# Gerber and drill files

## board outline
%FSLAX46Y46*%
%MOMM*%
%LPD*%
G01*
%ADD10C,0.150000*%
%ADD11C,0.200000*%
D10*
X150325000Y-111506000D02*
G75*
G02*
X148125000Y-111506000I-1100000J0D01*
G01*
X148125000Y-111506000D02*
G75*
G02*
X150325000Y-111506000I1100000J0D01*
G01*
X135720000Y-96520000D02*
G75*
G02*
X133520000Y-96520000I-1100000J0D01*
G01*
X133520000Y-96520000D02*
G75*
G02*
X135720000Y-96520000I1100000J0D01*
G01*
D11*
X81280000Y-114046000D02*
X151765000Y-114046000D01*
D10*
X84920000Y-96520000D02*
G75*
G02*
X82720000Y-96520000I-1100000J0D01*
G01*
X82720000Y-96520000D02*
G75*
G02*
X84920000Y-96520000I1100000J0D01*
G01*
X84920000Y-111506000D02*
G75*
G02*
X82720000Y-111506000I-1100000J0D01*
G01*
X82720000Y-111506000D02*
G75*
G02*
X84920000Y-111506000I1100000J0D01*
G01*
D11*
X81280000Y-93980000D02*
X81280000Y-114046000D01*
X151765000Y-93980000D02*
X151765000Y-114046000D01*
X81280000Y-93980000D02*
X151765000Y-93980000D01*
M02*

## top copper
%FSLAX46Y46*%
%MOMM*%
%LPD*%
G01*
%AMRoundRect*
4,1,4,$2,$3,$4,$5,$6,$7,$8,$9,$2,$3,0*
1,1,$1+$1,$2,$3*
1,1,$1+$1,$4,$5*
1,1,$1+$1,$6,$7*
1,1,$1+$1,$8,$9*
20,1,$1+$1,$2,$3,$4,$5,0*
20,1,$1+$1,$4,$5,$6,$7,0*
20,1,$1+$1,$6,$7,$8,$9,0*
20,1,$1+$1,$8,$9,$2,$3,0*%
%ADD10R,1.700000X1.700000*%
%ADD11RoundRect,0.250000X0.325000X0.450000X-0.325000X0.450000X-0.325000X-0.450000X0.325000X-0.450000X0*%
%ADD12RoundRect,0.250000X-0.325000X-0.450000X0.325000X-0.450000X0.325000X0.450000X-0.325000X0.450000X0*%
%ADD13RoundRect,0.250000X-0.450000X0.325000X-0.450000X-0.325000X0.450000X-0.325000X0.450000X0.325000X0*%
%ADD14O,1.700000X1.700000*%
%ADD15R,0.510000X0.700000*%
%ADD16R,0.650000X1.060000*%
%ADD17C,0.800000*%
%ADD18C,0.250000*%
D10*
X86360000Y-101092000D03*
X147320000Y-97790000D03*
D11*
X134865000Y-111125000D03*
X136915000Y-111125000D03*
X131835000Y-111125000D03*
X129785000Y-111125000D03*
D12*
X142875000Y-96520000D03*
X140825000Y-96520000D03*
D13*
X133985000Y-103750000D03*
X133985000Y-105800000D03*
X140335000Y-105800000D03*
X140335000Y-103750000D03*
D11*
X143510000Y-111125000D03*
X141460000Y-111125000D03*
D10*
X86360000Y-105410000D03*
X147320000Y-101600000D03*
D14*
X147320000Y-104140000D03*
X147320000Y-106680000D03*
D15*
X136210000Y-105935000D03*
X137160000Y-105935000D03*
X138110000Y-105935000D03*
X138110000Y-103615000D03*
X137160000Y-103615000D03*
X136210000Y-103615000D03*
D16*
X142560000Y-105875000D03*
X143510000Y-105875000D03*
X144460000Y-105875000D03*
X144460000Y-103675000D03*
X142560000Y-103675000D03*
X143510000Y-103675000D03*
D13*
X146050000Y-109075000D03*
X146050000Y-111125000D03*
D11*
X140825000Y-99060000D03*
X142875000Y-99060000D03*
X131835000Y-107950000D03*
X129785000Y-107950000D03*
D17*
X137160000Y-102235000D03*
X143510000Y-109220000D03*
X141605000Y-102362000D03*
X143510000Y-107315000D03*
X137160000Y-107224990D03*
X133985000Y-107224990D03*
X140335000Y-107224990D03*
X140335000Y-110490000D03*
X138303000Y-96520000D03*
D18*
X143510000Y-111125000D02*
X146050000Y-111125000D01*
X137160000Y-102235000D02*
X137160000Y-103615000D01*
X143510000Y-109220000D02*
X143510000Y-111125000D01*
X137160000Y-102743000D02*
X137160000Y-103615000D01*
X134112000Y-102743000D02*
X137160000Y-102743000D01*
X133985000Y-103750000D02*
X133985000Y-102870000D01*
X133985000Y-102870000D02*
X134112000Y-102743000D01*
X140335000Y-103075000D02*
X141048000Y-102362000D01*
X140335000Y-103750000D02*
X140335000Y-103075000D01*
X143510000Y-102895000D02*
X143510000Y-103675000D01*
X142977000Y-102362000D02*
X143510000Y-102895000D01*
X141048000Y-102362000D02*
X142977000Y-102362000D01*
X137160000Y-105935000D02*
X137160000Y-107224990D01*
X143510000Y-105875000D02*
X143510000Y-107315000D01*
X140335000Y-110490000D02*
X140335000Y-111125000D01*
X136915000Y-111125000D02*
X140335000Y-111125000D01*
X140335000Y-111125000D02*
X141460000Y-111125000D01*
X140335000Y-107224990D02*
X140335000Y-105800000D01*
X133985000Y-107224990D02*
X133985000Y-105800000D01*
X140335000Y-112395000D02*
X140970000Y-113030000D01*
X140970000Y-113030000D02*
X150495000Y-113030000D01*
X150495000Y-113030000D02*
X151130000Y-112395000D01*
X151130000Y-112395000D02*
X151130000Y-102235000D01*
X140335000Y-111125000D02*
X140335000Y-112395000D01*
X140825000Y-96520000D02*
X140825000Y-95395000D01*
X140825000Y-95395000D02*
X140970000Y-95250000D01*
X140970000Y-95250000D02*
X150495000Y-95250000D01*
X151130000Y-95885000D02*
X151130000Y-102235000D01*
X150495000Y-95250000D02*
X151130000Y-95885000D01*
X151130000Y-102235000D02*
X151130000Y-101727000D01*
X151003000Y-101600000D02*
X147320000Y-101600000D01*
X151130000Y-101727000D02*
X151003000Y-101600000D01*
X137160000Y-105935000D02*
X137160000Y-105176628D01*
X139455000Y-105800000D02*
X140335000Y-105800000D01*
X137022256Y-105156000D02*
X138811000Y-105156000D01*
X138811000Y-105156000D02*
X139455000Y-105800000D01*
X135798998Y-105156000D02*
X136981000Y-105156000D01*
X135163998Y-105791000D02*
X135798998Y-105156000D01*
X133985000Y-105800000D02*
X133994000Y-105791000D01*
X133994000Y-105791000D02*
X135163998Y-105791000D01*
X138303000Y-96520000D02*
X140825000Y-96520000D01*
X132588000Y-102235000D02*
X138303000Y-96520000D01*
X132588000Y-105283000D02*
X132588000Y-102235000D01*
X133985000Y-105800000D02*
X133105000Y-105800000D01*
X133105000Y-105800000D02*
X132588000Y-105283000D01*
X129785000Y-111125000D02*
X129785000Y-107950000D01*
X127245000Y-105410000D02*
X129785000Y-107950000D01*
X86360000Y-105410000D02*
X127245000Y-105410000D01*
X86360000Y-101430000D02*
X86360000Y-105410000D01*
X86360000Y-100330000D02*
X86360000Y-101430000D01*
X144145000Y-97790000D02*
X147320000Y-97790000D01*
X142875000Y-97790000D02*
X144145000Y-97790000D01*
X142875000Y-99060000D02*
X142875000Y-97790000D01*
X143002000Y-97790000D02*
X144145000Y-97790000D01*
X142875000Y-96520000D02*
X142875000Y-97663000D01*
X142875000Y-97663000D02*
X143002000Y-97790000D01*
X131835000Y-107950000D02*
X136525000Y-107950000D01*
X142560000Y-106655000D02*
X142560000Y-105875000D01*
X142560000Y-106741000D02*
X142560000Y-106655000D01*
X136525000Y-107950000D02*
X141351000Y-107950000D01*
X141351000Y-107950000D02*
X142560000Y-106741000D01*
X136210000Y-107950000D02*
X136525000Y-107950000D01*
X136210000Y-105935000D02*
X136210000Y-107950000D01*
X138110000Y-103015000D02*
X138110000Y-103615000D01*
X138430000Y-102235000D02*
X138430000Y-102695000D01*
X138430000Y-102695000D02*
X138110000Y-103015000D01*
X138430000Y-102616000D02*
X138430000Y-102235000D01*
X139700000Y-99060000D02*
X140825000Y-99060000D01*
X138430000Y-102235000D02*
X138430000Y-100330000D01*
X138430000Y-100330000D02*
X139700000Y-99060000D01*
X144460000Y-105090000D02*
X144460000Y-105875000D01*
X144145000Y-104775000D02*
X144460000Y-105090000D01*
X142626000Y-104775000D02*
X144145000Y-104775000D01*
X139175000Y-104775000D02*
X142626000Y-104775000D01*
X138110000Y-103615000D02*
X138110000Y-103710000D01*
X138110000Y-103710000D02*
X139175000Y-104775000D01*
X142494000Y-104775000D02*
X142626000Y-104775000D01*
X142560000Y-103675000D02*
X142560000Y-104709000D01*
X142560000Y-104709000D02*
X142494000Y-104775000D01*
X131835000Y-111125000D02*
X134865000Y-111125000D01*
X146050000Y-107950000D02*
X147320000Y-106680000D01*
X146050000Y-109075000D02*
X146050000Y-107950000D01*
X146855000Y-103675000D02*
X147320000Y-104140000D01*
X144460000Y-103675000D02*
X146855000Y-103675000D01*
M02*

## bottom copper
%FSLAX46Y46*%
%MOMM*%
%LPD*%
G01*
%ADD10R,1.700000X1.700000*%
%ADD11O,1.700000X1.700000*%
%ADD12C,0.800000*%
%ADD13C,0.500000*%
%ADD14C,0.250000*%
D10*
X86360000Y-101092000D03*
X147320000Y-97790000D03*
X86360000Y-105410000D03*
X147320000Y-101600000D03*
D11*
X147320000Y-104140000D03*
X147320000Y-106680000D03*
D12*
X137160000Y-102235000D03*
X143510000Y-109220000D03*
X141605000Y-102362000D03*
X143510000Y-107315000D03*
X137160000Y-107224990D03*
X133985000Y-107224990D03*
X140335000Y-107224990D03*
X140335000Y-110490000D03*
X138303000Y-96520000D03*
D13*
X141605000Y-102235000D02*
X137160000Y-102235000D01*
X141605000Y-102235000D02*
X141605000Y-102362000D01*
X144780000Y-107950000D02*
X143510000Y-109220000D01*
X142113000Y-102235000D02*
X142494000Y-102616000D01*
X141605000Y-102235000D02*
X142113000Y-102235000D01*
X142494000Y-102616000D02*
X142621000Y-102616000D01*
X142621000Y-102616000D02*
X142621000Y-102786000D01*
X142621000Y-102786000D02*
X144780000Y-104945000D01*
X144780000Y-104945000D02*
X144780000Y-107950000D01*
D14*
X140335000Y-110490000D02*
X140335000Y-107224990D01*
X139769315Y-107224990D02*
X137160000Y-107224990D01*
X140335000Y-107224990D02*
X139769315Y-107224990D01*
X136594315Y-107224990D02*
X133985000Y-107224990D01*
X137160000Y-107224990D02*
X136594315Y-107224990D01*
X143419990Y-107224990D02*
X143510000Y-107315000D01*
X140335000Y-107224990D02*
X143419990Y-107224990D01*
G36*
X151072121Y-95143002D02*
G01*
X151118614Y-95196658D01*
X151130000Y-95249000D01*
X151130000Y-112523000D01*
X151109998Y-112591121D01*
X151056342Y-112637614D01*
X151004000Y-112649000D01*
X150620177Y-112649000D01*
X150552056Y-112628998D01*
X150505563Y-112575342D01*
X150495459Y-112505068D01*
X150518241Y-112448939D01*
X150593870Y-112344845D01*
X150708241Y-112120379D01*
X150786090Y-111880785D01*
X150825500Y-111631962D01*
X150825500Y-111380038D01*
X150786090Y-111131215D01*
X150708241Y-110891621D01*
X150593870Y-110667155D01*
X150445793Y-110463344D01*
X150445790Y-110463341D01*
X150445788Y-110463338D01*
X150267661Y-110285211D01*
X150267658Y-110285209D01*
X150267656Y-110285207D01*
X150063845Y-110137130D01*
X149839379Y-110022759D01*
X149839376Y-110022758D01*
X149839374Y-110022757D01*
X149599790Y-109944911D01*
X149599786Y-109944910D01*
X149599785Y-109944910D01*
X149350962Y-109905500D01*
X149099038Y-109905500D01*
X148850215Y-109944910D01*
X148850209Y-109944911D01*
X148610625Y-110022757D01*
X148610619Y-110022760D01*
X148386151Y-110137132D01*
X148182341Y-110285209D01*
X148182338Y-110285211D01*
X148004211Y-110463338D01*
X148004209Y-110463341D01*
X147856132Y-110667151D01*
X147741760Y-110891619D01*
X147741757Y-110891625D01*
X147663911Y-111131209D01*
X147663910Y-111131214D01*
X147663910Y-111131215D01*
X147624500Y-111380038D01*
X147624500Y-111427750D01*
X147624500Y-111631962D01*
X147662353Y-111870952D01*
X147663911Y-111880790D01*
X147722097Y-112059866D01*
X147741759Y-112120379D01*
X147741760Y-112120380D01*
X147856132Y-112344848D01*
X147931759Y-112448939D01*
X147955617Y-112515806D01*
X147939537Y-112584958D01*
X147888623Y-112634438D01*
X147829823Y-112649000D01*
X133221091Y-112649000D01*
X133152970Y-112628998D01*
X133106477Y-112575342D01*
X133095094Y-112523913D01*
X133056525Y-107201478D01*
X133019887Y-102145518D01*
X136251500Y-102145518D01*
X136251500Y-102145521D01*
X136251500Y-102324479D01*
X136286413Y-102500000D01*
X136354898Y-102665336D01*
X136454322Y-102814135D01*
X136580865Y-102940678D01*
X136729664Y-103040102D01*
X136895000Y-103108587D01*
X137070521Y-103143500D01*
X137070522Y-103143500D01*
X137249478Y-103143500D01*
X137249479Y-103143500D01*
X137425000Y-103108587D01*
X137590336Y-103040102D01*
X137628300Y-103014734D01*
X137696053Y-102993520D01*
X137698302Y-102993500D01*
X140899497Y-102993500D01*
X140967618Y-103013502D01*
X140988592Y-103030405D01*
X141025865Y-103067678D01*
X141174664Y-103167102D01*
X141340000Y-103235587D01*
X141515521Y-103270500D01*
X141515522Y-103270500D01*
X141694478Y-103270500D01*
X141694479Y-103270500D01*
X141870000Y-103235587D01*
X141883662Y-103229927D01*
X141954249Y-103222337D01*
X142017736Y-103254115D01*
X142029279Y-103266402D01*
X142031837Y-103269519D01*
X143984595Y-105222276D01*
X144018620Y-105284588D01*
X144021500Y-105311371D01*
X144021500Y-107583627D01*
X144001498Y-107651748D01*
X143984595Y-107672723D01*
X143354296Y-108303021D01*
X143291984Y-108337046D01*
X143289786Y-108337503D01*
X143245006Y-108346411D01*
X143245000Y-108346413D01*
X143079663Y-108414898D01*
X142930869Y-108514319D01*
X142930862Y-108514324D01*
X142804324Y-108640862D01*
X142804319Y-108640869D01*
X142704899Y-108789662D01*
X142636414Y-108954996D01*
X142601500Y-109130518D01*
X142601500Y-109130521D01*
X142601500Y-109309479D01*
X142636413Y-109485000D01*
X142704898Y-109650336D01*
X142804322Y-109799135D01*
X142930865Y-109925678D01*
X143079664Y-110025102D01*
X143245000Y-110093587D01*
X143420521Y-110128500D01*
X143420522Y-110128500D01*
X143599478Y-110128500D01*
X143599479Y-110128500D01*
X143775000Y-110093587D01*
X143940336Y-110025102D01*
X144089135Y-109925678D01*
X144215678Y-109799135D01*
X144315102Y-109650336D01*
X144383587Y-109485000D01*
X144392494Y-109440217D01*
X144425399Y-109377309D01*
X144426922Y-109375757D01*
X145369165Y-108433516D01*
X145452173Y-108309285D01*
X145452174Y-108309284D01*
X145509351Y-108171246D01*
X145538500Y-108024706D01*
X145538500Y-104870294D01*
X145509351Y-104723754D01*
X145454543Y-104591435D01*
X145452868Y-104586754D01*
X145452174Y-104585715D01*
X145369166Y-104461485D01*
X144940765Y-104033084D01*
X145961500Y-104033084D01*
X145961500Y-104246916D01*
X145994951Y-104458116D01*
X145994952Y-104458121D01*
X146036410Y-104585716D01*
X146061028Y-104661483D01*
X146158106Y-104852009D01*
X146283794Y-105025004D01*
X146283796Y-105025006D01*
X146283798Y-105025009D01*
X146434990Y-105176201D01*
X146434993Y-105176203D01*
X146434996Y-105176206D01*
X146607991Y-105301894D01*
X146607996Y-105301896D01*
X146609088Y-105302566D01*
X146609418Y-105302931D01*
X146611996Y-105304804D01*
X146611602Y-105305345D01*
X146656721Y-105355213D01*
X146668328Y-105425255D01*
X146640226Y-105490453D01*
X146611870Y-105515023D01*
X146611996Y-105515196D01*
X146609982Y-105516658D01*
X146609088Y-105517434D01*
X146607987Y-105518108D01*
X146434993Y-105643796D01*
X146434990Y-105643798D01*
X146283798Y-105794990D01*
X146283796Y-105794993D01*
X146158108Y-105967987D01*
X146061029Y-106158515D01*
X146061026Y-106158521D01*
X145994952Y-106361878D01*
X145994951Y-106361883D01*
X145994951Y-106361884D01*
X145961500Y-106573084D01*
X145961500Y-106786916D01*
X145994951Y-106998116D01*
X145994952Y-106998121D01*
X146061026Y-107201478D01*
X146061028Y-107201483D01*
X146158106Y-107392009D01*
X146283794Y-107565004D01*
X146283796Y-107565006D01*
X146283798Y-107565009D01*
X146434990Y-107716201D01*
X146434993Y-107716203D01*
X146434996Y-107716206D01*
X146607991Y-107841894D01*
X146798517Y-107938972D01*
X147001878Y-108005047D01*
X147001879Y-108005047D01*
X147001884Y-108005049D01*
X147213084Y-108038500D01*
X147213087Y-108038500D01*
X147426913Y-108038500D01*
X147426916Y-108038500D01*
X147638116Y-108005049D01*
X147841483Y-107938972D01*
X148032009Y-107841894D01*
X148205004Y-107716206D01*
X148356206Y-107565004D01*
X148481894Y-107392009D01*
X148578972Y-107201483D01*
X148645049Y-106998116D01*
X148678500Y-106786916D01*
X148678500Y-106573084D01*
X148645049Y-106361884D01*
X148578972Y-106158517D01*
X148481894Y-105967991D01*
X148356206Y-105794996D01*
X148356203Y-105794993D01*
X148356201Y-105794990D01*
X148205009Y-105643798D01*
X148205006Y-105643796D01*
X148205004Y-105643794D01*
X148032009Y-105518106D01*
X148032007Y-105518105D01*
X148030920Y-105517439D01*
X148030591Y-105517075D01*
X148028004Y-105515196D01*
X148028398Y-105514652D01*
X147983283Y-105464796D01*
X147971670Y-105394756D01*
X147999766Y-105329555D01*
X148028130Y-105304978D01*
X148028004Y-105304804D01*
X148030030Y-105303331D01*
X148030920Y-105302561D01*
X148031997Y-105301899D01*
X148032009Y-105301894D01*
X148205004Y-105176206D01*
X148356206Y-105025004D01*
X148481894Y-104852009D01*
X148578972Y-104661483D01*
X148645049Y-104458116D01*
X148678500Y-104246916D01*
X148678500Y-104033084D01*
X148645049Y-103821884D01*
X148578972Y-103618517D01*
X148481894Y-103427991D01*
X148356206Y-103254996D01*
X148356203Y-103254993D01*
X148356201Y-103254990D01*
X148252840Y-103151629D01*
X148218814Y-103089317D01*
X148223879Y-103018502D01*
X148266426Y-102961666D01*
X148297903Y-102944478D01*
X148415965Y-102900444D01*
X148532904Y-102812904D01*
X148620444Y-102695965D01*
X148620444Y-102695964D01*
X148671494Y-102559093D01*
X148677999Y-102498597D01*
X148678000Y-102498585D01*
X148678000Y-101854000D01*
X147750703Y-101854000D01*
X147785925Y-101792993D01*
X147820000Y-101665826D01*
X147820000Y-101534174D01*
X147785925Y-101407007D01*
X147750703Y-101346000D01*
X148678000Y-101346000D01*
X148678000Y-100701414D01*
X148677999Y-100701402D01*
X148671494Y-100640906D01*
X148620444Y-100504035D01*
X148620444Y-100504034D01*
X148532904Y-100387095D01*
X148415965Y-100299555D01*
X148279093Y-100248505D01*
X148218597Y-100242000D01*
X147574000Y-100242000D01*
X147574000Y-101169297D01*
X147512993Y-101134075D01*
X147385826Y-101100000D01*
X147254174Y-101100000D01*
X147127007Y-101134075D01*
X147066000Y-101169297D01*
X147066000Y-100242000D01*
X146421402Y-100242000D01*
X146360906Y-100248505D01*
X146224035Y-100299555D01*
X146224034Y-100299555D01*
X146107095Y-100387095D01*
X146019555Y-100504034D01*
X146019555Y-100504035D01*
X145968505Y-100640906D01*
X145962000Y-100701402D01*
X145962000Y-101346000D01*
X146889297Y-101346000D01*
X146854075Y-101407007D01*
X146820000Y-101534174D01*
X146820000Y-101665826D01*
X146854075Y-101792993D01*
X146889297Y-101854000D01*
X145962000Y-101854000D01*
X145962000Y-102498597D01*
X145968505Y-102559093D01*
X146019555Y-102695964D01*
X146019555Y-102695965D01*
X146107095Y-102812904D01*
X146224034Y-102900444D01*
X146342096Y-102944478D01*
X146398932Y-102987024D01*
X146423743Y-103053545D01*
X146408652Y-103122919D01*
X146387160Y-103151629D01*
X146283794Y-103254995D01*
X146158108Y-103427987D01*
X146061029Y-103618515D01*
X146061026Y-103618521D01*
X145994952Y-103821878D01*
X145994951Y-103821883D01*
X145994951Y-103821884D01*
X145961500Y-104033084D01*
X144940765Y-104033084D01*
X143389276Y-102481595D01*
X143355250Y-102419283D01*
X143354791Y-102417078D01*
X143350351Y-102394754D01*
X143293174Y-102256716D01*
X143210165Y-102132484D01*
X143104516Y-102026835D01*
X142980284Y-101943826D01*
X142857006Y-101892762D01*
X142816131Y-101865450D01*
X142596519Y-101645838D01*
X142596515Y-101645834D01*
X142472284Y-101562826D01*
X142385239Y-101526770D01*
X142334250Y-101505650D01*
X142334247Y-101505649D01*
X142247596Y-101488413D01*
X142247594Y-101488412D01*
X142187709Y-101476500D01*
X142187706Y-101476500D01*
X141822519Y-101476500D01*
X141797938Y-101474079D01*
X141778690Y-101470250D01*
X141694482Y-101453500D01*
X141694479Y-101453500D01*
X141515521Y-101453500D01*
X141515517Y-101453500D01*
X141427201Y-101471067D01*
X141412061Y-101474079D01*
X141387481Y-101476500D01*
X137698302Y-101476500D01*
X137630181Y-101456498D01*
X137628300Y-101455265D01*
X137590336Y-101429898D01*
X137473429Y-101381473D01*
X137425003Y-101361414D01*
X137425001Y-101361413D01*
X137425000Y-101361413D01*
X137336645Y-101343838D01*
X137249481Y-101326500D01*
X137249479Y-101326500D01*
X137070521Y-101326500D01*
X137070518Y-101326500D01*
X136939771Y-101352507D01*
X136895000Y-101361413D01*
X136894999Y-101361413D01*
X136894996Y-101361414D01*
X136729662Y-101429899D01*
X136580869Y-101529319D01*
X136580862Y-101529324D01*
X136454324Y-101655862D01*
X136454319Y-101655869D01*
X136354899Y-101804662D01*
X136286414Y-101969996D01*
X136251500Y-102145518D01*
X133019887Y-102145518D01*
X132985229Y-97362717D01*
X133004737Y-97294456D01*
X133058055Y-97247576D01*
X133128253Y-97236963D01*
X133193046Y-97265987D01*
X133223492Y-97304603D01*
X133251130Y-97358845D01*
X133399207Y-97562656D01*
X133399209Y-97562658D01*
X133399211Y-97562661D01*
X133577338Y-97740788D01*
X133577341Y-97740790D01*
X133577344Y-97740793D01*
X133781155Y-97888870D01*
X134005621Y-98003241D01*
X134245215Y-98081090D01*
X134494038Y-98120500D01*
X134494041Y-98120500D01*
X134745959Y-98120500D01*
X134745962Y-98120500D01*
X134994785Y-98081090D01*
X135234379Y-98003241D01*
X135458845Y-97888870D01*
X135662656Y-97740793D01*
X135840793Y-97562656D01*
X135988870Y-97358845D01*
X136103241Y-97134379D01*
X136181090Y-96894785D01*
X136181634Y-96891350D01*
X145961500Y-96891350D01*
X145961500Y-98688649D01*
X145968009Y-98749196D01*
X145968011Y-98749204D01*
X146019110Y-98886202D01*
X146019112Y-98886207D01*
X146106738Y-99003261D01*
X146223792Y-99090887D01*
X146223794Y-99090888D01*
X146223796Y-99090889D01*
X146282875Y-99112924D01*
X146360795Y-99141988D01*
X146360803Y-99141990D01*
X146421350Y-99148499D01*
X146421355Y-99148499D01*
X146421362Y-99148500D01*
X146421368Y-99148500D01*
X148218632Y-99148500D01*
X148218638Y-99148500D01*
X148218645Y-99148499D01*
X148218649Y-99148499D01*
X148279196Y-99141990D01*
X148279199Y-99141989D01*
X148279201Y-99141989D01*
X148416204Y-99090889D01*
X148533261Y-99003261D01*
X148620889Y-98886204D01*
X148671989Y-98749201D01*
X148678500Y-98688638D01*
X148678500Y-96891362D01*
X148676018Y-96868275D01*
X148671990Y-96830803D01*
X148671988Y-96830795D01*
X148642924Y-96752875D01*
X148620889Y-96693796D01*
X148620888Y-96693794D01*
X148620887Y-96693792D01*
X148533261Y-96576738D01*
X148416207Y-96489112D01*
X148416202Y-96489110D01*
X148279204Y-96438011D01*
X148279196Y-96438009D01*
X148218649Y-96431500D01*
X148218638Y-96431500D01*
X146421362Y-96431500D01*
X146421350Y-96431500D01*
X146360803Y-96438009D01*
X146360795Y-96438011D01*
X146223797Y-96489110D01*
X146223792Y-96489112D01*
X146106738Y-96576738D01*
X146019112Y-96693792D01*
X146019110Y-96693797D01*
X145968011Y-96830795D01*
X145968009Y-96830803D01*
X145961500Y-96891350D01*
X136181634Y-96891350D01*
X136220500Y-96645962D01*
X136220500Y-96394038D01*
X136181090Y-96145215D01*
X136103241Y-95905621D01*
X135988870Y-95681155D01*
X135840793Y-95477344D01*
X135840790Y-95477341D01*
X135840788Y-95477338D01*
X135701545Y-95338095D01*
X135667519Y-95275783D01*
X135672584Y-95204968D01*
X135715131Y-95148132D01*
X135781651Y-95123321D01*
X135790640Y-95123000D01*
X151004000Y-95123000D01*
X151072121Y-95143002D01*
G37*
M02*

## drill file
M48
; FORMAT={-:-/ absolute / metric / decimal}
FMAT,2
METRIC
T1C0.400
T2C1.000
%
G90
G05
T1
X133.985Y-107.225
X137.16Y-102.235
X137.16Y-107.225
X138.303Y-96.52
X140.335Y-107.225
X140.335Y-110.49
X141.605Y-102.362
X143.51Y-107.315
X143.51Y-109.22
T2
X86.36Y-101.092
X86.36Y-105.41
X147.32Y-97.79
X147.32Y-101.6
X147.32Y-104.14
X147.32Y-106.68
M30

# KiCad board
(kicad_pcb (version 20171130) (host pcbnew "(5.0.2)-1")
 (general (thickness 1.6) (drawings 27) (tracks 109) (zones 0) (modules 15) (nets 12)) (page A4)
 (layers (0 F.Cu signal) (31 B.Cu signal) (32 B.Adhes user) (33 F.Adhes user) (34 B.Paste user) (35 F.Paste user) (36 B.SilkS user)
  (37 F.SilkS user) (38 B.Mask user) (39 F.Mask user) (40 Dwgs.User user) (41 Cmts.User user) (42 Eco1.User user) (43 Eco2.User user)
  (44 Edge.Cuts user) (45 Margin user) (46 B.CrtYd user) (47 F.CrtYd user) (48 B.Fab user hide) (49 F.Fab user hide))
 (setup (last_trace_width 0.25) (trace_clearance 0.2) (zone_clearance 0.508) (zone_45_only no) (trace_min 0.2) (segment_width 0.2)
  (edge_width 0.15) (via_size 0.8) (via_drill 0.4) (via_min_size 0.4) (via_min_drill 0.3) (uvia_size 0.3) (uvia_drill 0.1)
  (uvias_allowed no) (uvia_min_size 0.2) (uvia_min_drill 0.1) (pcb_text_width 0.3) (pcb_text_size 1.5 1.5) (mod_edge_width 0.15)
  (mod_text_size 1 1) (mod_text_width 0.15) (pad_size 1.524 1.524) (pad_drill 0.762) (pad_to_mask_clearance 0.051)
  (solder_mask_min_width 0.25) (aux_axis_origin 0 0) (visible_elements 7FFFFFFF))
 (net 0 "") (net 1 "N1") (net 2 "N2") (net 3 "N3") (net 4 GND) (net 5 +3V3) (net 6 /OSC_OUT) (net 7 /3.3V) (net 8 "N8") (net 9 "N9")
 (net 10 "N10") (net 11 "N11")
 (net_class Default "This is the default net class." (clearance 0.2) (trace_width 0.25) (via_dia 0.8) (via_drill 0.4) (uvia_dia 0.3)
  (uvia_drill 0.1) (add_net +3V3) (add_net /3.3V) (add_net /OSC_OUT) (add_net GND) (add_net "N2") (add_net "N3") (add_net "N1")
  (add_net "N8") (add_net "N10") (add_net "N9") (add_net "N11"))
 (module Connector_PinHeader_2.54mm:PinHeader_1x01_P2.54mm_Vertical (layer F.Cu) (at 86.36 101.092 180)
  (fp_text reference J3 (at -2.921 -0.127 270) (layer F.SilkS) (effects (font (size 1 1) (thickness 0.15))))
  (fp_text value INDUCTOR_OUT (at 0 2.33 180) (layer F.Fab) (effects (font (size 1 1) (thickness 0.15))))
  (pad 1 thru_hole rect (at 0 0 180) (size 1.7 1.7) (drill 1) (layers *.Cu *.Mask) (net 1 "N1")))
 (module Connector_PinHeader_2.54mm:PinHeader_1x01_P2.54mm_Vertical (layer F.Cu) (at 147.32 97.79)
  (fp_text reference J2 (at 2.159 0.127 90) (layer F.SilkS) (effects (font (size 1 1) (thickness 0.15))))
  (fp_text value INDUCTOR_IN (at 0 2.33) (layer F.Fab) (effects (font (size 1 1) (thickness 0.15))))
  (pad 1 thru_hole rect (at 0 0) (size 1.7 1.7) (drill 1) (layers *.Cu *.Mask) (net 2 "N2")))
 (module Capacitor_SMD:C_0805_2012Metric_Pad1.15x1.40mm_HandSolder (layer F.Cu) (at 135.89 111.125 180)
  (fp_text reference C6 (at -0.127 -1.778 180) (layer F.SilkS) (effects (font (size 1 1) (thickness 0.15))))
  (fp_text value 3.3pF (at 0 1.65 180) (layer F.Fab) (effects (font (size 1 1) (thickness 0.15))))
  (pad 2 smd roundrect (at 1.025 0 180) (size 1.15 1.4) (layers F.Cu F.Paste F.Mask) (roundrect_rratio 0.217391) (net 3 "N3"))
  (pad 1 smd roundrect (at -1.025 0 180) (size 1.15 1.4) (layers F.Cu F.Paste F.Mask) (roundrect_rratio 0.217391) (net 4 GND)))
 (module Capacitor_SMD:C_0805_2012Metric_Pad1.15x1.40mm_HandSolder (layer F.Cu) (at 130.81 111.125 180)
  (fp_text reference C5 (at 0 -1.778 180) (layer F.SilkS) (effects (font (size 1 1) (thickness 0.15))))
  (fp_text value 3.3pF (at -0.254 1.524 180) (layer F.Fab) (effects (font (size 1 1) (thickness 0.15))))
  (pad 1 smd roundrect (at -1.025 0 180) (size 1.15 1.4) (layers F.Cu F.Paste F.Mask) (roundrect_rratio 0.217391) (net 3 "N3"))
  (pad 2 smd roundrect (at 1.025 0 180) (size 1.15 1.4) (layers F.Cu F.Paste F.Mask) (roundrect_rratio 0.217391) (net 1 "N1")))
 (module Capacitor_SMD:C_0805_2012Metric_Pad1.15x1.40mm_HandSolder (layer F.Cu) (at 141.85 96.52)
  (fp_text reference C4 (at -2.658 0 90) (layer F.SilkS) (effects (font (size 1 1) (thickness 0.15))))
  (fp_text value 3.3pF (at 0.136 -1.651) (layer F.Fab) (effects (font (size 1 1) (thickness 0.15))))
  (pad 2 smd roundrect (at 1.025 0) (size 1.15 1.4) (layers F.Cu F.Paste F.Mask) (roundrect_rratio 0.217391) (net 2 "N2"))
  (pad 1 smd roundrect (at -1.025 0) (size 1.15 1.4) (layers F.Cu F.Paste F.Mask) (roundrect_rratio 0.217391) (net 4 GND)))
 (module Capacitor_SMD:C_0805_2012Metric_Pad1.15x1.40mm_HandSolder (layer F.Cu) (at 133.985 104.775 270)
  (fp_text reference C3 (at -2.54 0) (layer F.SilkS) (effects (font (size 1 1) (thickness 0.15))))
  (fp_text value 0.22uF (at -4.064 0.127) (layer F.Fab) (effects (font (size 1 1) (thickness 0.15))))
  (pad 1 smd roundrect (at -1.025 0 270) (size 1.15 1.4) (layers F.Cu F.Paste F.Mask) (roundrect_rratio 0.217391) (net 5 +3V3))
  (pad 2 smd roundrect (at 1.025 0 270) (size 1.15 1.4) (layers F.Cu F.Paste F.Mask) (roundrect_rratio 0.217391) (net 4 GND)))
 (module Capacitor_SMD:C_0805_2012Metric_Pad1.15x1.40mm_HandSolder (layer F.Cu) (at 140.335 104.775 270)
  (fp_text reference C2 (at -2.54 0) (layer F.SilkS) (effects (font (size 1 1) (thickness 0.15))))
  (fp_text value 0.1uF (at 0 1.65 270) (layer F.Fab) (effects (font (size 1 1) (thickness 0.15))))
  (pad 2 smd roundrect (at 1.025 0 270) (size 1.15 1.4) (layers F.Cu F.Paste F.Mask) (roundrect_rratio 0.217391) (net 4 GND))
  (pad 1 smd roundrect (at -1.025 0 270) (size 1.15 1.4) (layers F.Cu F.Paste F.Mask) (roundrect_rratio 0.217391) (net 5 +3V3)))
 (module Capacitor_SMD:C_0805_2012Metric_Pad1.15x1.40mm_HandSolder (layer F.Cu) (at 142.485 111.125 180)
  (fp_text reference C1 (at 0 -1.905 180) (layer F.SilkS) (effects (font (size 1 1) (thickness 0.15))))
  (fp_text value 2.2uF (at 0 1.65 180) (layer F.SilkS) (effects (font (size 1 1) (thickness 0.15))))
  (pad 1 smd roundrect (at -1.025 0 180) (size 1.15 1.4) (layers F.Cu F.Paste F.Mask) (roundrect_rratio 0.217391) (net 5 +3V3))
  (pad 2 smd roundrect (at 1.025 0 180) (size 1.15 1.4) (layers F.Cu F.Paste F.Mask) (roundrect_rratio 0.217391) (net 4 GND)))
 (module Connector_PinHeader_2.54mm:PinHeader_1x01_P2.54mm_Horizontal (layer F.Cu) (at 86.36 105.41 180)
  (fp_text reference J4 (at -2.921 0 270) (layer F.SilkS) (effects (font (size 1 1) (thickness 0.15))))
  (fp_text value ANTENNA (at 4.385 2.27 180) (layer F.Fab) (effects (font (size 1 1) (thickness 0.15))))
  (pad 1 thru_hole rect (at 0 0 180) (size 1.7 1.7) (drill 1) (layers *.Cu *.Mask) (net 1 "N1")))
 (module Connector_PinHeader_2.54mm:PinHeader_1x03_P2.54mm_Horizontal (layer F.Cu) (at 147.32 101.6)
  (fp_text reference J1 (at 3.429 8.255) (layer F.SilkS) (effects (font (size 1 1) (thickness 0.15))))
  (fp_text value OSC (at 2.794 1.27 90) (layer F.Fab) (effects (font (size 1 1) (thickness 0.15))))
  (pad 1 thru_hole rect (at 0 0) (size 1.7 1.7) (drill 1) (layers *.Cu *.Mask) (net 4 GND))
  (pad 2 thru_hole oval (at 0 2.54) (size 1.7 1.7) (drill 1) (layers *.Cu *.Mask) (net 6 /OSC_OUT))
  (pad 3 thru_hole oval (at 0 5.08) (size 1.7 1.7) (drill 1) (layers *.Cu *.Mask) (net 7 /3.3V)))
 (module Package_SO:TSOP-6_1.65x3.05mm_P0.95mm (layer F.Cu) (at 137.16 104.775 90)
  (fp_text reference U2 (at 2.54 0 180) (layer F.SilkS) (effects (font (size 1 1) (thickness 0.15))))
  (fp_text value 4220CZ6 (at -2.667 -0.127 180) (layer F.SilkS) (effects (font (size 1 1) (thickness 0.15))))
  (pad 1 smd rect (at -1.16 -0.95 90) (size 0.7 0.51) (layers F.Cu F.Paste F.Mask) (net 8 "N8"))
  (pad 2 smd rect (at -1.16 0 90) (size 0.7 0.51) (layers F.Cu F.Paste F.Mask) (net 4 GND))
  (pad 3 smd rect (at -1.16 0.95 90) (size 0.7 0.51) (layers F.Cu F.Paste F.Mask) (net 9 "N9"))
  (pad 4 smd rect (at 1.16 0.95 90) (size 0.7 0.51) (layers F.Cu F.Paste F.Mask) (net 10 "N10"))
  (pad 5 smd rect (at 1.16 0 90) (size 0.7 0.51) (layers F.Cu F.Paste F.Mask) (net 5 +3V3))
  (pad 6 smd rect (at 1.16 -0.95 90) (size 0.7 0.51) (layers F.Cu F.Paste F.Mask) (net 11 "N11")))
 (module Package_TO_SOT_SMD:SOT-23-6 (layer F.Cu) (at 143.51 104.775 90)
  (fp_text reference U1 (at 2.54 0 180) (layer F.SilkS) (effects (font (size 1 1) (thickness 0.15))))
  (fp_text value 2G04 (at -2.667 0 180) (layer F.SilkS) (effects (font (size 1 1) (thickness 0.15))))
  (pad 1 smd rect (at -1.1 -0.95 90) (size 1.06 0.65) (layers F.Cu F.Paste F.Mask) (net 8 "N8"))
  (pad 2 smd rect (at -1.1 0 90) (size 1.06 0.65) (layers F.Cu F.Paste F.Mask) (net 4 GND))
  (pad 3 smd rect (at -1.1 0.95 90) (size 1.06 0.65) (layers F.Cu F.Paste F.Mask) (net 10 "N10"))
  (pad 4 smd rect (at 1.1 0.95 90) (size 1.06 0.65) (layers F.Cu F.Paste F.Mask) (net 6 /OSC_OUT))
  (pad 6 smd rect (at 1.1 -0.95 90) (size 1.06 0.65) (layers F.Cu F.Paste F.Mask) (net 10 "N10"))
  (pad 5 smd rect (at 1.1 0 90) (size 1.06 0.65) (layers F.Cu F.Paste F.Mask) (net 5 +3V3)))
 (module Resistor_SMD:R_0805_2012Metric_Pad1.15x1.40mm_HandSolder (layer F.Cu) (at 146.05 110.1 270)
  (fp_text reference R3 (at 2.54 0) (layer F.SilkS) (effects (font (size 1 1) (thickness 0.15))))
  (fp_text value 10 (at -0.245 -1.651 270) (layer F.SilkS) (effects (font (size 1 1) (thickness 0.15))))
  (pad 1 smd roundrect (at -1.025 0 270) (size 1.15 1.4) (layers F.Cu F.Paste F.Mask) (roundrect_rratio 0.217391) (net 7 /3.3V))
  (pad 2 smd roundrect (at 1.025 0 270) (size 1.15 1.4) (layers F.Cu F.Paste F.Mask) (roundrect_rratio 0.217391) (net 5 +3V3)))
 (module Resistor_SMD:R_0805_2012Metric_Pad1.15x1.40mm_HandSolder (layer F.Cu) (at 141.85 99.06 180)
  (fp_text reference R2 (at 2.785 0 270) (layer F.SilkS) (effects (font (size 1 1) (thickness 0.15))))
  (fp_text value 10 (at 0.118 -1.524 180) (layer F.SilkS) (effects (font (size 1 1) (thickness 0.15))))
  (pad 2 smd roundrect (at 1.025 0 180) (size 1.15 1.4) (layers F.Cu F.Paste F.Mask) (roundrect_rratio 0.217391) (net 10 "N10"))
  (pad 1 smd roundrect (at -1.025 0 180) (size 1.15 1.4) (layers F.Cu F.Paste F.Mask) (roundrect_rratio 0.217391) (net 2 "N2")))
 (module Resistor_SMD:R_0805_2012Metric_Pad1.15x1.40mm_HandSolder (layer F.Cu) (at 130.81 107.95 180)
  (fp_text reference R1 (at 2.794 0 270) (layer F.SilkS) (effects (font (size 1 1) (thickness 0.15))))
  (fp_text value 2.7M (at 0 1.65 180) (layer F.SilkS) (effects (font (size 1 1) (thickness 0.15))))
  (pad 1 smd roundrect (at -1.025 0 180) (size 1.15 1.4) (layers F.Cu F.Paste F.Mask) (roundrect_rratio 0.217391) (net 8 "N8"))
  (pad 2 smd roundrect (at 1.025 0 180) (size 1.15 1.4) (layers F.Cu F.Paste F.Mask) (roundrect_rratio 0.217391) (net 1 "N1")))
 (gr_circle (center 149.225 111.506) (end 150.325 111.506) (layer Edge.Cuts) (width 0.15))
 (gr_circle (center 134.62 96.52) (end 135.72 96.52) (layer Edge.Cuts) (width 0.15))
 (gr_line (start 81.28 114.046) (end 151.765 114.046) (layer Edge.Cuts) (width 0.2))
 (gr_circle (center 83.82 96.52) (end 84.92 96.52) (layer Edge.Cuts) (width 0.15))
 (gr_circle (center 83.82 111.506) (end 84.92 111.506) (layer Edge.Cuts) (width 0.15))
 (gr_line (start 81.28 93.98) (end 81.28 114.046) (layer Edge.Cuts) (width 0.2))
 (gr_line (start 151.765 93.98) (end 151.765 114.046) (layer Edge.Cuts) (width 0.2))
 (gr_line (start 81.28 93.98) (end 151.765 93.98) (layer Edge.Cuts) (width 0.2))
 (via (at 137.16 102.235) (size 0.8) (drill 0.4) (layers F.Cu B.Cu) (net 5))
 (segment (start 143.51 111.125) (end 146.05 111.125) (width 0.25) (layer F.Cu) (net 5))
 (via (at 143.51 109.22) (size 0.8) (drill 0.4) (layers F.Cu B.Cu) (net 5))
 (segment (start 137.16 102.235) (end 137.16 103.615) (width 0.25) (layer F.Cu) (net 5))
 (segment (start 143.51 109.22) (end 143.51 111.125) (width 0.25) (layer F.Cu) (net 5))
 (segment (start 141.605 102.235) (end 137.16 102.235) (width 0.5) (layer B.Cu) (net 5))
 (segment (start 137.16 102.743) (end 137.16 103.615) (width 0.25) (layer F.Cu) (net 5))
 (segment (start 134.112 102.743) (end 137.16 102.743) (width 0.25) (layer F.Cu) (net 5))
 (segment (start 133.985 103.75) (end 133.985 102.87) (width 0.25) (layer F.Cu) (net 5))
 (segment (start 133.985 102.87) (end 134.112 102.743) (width 0.25) (layer F.Cu) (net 5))
 (segment (start 140.335 103.075) (end 141.048 102.362) (width 0.25) (layer F.Cu) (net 5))
 (segment (start 140.335 103.75) (end 140.335 103.075) (width 0.25) (layer F.Cu) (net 5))
 (segment (start 143.51 102.895) (end 143.51 103.675) (width 0.25) (layer F.Cu) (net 5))
 (segment (start 142.977 102.362) (end 143.51 102.895) (width 0.25) (layer F.Cu) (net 5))
 (segment (start 141.048 102.362) (end 142.977 102.362) (width 0.25) (layer F.Cu) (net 5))
 (segment (start 141.605 102.235) (end 141.605 102.362) (width 0.5) (layer B.Cu) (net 5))
 (via (at 141.605 102.362) (size 0.8) (drill 0.4) (layers F.Cu B.Cu) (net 5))
 (segment (start 144.78 107.95) (end 143.51 109.22) (width 0.5) (layer B.Cu) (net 5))
 (segment (start 142.113 102.235) (end 142.494 102.616) (width 0.5) (layer B.Cu) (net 5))
 (segment (start 141.605 102.235) (end 142.113 102.235) (width 0.5) (layer B.Cu) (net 5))
 (segment (start 142.494 102.616) (end 142.621 102.616) (width 0.5) (layer B.Cu) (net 5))
 (segment (start 142.621 102.616) (end 142.621 102.786) (width 0.5) (layer B.Cu) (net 5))
 (segment (start 142.621 102.786) (end 144.78 104.945) (width 0.5) (layer B.Cu) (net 5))
 (segment (start 144.78 104.945) (end 144.78 107.95) (width 0.5) (layer B.Cu) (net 5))
 (via (at 143.51 107.315) (size 0.8) (drill 0.4) (layers F.Cu B.Cu) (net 4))
 (via (at 137.16 107.22499) (size 0.8) (drill 0.4) (layers F.Cu B.Cu) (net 4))
 (segment (start 137.16 105.935) (end 137.16 107.22499) (width 0.25) (layer F.Cu) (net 4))
 (segment (start 143.51 105.875) (end 143.51 107.315) (width 0.25) (layer F.Cu) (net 4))
 (via (at 133.985 107.22499) (size 0.8) (drill 0.4) (layers F.Cu B.Cu) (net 4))
 (via (at 140.335 107.22499) (size 0.8) (drill 0.4) (layers F.Cu B.Cu) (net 4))
 (via (at 140.335 110.49) (size 0.8) (drill 0.4) (layers F.Cu B.Cu) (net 4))
 (segment (start 140.335 110.49) (end 140.335 111.125) (width 0.25) (layer F.Cu) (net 4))
 (segment (start 136.915 111.125) (end 140.335 111.125) (width 0.25) (layer F.Cu) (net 4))
 (segment (start 140.335 111.125) (end 141.46 111.125) (width 0.25) (layer F.Cu) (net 4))
 (segment (start 140.335 107.22499) (end 140.335 105.8) (width 0.25) (layer F.Cu) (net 4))
 (segment (start 133.985 107.22499) (end 133.985 105.8) (width 0.25) (layer F.Cu) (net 4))
 (segment (start 140.335 110.49) (end 140.335 107.22499) (width 0.25) (layer B.Cu) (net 4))
 (segment (start 139.769315 107.22499) (end 137.16 107.22499) (width 0.25) (layer B.Cu) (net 4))
 (segment (start 140.335 107.22499) (end 139.769315 107.22499) (width 0.25) (layer B.Cu) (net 4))
 (segment (start 136.594315 107.22499) (end 133.985 107.22499) (width 0.25) (layer B.Cu) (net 4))
 (segment (start 137.16 107.22499) (end 136.594315 107.22499) (width 0.25) (layer B.Cu) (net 4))
 (segment (start 143.41999 107.22499) (end 143.51 107.315) (width 0.25) (layer B.Cu) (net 4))
 (segment (start 140.335 107.22499) (end 143.41999 107.22499) (width 0.25) (layer B.Cu) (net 4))
 (segment (start 140.335 112.395) (end 140.97 113.03) (width 0.25) (layer F.Cu) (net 4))
 (segment (start 140.97 113.03) (end 150.495 113.03) (width 0.25) (layer F.Cu) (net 4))
 (segment (start 150.495 113.03) (end 151.13 112.395) (width 0.25) (layer F.Cu) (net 4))
 (segment (start 151.13 112.395) (end 151.13 102.235) (width 0.25) (layer F.Cu) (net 4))
 (segment (start 140.335 111.125) (end 140.335 112.395) (width 0.25) (layer F.Cu) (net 4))
 (segment (start 140.825 96.52) (end 140.825 95.395) (width 0.25) (layer F.Cu) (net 4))
 (segment (start 140.825 95.395) (end 140.97 95.25) (width 0.25) (layer F.Cu) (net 4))
 (segment (start 140.97 95.25) (end 150.495 95.25) (width 0.25) (layer F.Cu) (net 4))
 (segment (start 151.13 95.885) (end 151.13 102.235) (width 0.25) (layer F.Cu) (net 4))
 (segment (start 150.495 95.25) (end 151.13 95.885) (width 0.25) (layer F.Cu) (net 4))
 (segment (start 151.13 102.235) (end 151.13 101.727) (width 0.25) (layer F.Cu) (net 4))
 (segment (start 151.003 101.6) (end 147.32 101.6) (width 0.25) (layer F.Cu) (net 4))
 (segment (start 151.13 101.727) (end 151.003 101.6) (width 0.25) (layer F.Cu) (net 4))
 (segment (start 137.16 105.935) (end 137.16 105.176628) (width 0.25) (layer F.Cu) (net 4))
 (segment (start 139.455 105.8) (end 140.335 105.8) (width 0.25) (layer F.Cu) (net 4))
 (segment (start 137.022256 105.156) (end 138.811 105.156) (width 0.25) (layer F.Cu) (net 4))
 (segment (start 138.811 105.156) (end 139.455 105.8) (width 0.25) (layer F.Cu) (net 4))
 (segment (start 135.798998 105.156) (end 136.981 105.156) (width 0.25) (layer F.Cu) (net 4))
 (segment (start 135.163998 105.791) (end 135.798998 105.156) (width 0.25) (layer F.Cu) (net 4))
 (segment (start 133.985 105.8) (end 133.994 105.791) (width 0.25) (layer F.Cu) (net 4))
 (segment (start 133.994 105.791) (end 135.163998 105.791) (width 0.25) (layer F.Cu) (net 4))
 (segment (start 138.303 96.52) (end 140.825 96.52) (width 0.25) (layer F.Cu) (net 4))
 (segment (start 132.588 102.235) (end 138.303 96.52) (width 0.25) (layer F.Cu) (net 4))
 (segment (start 132.588 105.283) (end 132.588 102.235) (width 0.25) (layer F.Cu) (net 4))
 (segment (start 133.985 105.8) (end 133.105 105.8) (width 0.25) (layer F.Cu) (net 4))
 (segment (start 133.105 105.8) (end 132.588 105.283) (width 0.25) (layer F.Cu) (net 4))
 (via (at 138.303 96.52) (size 0.8) (drill 0.4) (layers F.Cu B.Cu) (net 4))
 (segment (start 129.785 111.125) (end 129.785 107.95) (width 0.25) (layer F.Cu) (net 1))
 (segment (start 127.245 105.41) (end 129.785 107.95) (width 0.25) (layer F.Cu) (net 1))
 (segment (start 86.36 105.41) (end 127.245 105.41) (width 0.25) (layer F.Cu) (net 1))
 (segment (start 86.36 101.43) (end 86.36 105.41) (width 0.25) (layer F.Cu) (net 1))
 (segment (start 86.36 100.33) (end 86.36 101.43) (width 0.25) (layer F.Cu) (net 1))
 (segment (start 144.145 97.79) (end 147.32 97.79) (width 0.25) (layer F.Cu) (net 2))
 (segment (start 142.875 97.79) (end 144.145 97.79) (width 0.25) (layer F.Cu) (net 2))
 (segment (start 142.875 99.06) (end 142.875 97.79) (width 0.25) (layer F.Cu) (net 2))
 (segment (start 143.002 97.79) (end 144.145 97.79) (width 0.25) (layer F.Cu) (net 2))
 (segment (start 142.875 96.52) (end 142.875 97.663) (width 0.25) (layer F.Cu) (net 2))
 (segment (start 142.875 97.663) (end 143.002 97.79) (width 0.25) (layer F.Cu) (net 2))
 (segment (start 131.835 107.95) (end 136.525 107.95) (width 0.25) (layer F.Cu) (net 8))
 (segment (start 142.56 106.655) (end 142.56 105.875) (width 0.25) (layer F.Cu) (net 8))
 (segment (start 142.56 106.741) (end 142.56 106.655) (width 0.25) (layer F.Cu) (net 8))
 (segment (start 136.525 107.95) (end 141.351 107.95) (width 0.25) (layer F.Cu) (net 8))
 (segment (start 141.351 107.95) (end 142.56 106.741) (width 0.25) (layer F.Cu) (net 8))
 (segment (start 136.21 107.95) (end 136.525 107.95) (width 0.25) (layer F.Cu) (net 8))
 (segment (start 136.21 105.935) (end 136.21 107.95) (width 0.25) (layer F.Cu) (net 8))
 (segment (start 138.11 103.015) (end 138.11 103.615) (width 0.25) (layer F.Cu) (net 10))
 (segment (start 138.43 102.235) (end 138.43 102.695) (width 0.25) (layer F.Cu) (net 10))
 (segment (start 138.43 102.695) (end 138.11 103.015) (width 0.25) (layer F.Cu) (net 10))
 (segment (start 138.43 102.616) (end 138.43 102.235) (width 0.25) (layer F.Cu) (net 10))
 (segment (start 139.7 99.06) (end 140.825 99.06) (width 0.25) (layer F.Cu) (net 10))
 (segment (start 138.43 102.235) (end 138.43 100.33) (width 0.25) (layer F.Cu) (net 10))
 (segment (start 138.43 100.33) (end 139.7 99.06) (width 0.25) (layer F.Cu) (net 10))
 (segment (start 144.46 105.09) (end 144.46 105.875) (width 0.25) (layer F.Cu) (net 10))
 (segment (start 144.145 104.775) (end 144.46 105.09) (width 0.25) (layer F.Cu) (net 10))
 (segment (start 142.626 104.775) (end 144.145 104.775) (width 0.25) (layer F.Cu) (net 10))
 (segment (start 139.175 104.775) (end 142.626 104.775) (width 0.25) (layer F.Cu) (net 10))
 (segment (start 138.11 103.615) (end 138.11 103.71) (width 0.25) (layer F.Cu) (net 10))
 (segment (start 138.11 103.71) (end 139.175 104.775) (width 0.25) (layer F.Cu) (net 10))
 (segment (start 142.494 104.775) (end 142.626 104.775) (width 0.25) (layer F.Cu) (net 10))
 (segment (start 142.56 103.675) (end 142.56 104.709) (width 0.25) (layer F.Cu) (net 10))
 (segment (start 142.56 104.709) (end 142.494 104.775) (width 0.25) (layer F.Cu) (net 10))
 (segment (start 131.835 111.125) (end 134.865 111.125) (width 0.25) (layer F.Cu) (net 3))
 (segment (start 146.05 107.95) (end 147.32 106.68) (width 0.25) (layer F.Cu) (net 7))
 (segment (start 146.05 109.075) (end 146.05 107.95) (width 0.25) (layer F.Cu) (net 7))
 (segment (start 146.855 103.675) (end 147.32 104.14) (width 0.25) (layer F.Cu) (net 6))
 (segment (start 144.46 103.675) (end 146.855 103.675) (width 0.25) (layer F.Cu) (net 6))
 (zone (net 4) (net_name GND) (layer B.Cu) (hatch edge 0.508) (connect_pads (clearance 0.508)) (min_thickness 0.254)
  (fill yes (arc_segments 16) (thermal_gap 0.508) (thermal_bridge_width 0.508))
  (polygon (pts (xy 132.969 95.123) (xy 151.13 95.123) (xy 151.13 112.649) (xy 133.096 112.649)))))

